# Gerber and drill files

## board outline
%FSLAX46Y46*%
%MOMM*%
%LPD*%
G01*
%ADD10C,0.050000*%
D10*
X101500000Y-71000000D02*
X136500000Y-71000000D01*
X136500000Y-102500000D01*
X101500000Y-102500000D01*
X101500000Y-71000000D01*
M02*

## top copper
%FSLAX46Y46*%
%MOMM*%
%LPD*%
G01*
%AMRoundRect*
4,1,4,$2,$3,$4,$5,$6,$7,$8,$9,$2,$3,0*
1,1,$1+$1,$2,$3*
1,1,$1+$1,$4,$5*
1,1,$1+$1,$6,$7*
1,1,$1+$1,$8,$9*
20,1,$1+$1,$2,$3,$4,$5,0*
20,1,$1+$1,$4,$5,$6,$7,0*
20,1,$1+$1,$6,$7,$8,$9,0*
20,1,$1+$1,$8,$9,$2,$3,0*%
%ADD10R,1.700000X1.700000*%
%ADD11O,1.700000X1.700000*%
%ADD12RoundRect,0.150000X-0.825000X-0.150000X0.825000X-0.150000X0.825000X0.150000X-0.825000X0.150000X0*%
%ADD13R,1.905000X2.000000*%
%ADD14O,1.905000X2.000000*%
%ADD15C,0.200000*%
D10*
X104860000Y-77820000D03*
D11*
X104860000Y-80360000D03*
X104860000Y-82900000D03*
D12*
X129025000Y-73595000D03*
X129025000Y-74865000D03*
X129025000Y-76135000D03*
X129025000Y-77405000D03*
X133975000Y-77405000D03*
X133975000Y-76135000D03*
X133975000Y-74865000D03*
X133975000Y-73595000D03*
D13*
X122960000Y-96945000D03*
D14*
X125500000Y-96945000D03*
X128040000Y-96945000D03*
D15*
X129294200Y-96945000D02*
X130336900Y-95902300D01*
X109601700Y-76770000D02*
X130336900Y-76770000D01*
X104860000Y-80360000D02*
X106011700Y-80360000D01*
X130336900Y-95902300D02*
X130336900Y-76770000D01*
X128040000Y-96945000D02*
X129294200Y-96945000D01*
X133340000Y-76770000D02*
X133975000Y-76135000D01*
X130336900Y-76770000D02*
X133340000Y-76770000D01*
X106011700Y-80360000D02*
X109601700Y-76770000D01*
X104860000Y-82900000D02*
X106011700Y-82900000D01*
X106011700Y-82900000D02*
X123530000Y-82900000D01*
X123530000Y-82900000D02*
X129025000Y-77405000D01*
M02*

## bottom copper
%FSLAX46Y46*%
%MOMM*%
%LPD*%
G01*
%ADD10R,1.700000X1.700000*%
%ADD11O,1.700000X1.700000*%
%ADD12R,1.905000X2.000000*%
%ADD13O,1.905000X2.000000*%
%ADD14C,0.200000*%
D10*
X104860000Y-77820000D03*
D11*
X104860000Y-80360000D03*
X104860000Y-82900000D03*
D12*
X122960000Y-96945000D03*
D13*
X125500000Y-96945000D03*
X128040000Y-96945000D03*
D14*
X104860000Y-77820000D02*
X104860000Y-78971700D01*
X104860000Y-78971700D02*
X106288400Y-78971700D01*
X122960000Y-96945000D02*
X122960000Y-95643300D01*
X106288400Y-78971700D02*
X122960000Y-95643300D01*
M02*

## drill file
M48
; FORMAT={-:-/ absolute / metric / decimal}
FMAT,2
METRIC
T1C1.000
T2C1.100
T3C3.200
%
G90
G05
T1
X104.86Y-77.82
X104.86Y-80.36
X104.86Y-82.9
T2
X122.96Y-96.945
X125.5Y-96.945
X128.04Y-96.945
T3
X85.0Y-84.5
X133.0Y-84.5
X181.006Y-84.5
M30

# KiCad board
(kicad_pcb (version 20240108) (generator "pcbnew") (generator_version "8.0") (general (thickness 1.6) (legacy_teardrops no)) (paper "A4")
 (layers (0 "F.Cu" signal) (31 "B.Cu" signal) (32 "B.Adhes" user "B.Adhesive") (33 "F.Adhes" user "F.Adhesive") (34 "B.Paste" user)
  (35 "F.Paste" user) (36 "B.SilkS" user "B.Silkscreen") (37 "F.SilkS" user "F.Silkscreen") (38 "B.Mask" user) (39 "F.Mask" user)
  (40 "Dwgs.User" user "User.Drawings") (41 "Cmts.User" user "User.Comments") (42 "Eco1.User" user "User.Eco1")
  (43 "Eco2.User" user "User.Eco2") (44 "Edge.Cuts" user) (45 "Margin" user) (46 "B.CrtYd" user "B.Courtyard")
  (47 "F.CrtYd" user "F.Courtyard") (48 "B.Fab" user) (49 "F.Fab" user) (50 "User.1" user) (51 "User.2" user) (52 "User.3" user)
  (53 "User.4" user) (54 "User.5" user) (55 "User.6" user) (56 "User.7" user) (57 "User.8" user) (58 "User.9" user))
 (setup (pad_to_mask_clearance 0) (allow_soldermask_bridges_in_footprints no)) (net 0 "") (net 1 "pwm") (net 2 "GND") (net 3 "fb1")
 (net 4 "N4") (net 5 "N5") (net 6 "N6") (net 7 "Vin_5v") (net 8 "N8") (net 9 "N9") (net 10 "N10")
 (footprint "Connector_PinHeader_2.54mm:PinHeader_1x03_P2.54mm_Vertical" (layer "F.Cu") (at 104.86 77.82)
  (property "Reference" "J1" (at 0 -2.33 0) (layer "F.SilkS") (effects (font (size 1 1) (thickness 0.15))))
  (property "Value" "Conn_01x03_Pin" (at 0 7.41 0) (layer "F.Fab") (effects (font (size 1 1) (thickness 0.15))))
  (pad "1" thru_hole rect (at 0 0) (size 1.7 1.7) (drill 1) (layers "*.Cu" "*.Mask") (remove_unused_layers no) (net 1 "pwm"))
  (pad "2" thru_hole oval (at 0 2.54) (size 1.7 1.7) (drill 1) (layers "*.Cu" "*.Mask") (remove_unused_layers no) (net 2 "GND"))
  (pad "3" thru_hole oval (at 0 5.08) (size 1.7 1.7) (drill 1) (layers "*.Cu" "*.Mask") (remove_unused_layers no) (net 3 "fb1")))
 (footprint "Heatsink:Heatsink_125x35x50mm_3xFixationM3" (layer "F.Cu") (at 133 84.5)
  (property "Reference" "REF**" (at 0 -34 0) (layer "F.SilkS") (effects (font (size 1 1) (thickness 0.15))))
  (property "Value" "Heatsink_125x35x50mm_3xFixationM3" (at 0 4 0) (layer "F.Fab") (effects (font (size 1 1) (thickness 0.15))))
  (pad "" np_thru_hole circle (at -48 0) (size 3.2 3.2) (drill 3.2) (layers "*.Cu" "*.SilkS" "*.Mask"))
  (pad "" np_thru_hole circle (at 0 0) (size 3.2 3.2) (drill 3.2) (layers "*.Cu" "*.SilkS" "*.Mask"))
  (pad "" np_thru_hole circle (at 48.006 0) (size 3.2 3.2) (drill 3.2) (layers "*.Cu" "*.SilkS" "*.Mask")))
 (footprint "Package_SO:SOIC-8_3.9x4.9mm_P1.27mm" (layer "F.Cu") (at 131.5 75.5)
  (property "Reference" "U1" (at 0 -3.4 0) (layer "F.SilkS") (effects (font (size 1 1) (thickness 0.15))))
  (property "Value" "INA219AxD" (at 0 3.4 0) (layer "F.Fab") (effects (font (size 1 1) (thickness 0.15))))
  (pad "1" smd roundrect (at -2.475 -1.905) (size 1.95 0.6) (layers "F.Cu" "F.Paste" "F.Mask") (roundrect_rratio 0.25) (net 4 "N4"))
  (pad "2" smd roundrect (at -2.475 -0.635) (size 1.95 0.6) (layers "F.Cu" "F.Paste" "F.Mask") (roundrect_rratio 0.25) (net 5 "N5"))
  (pad "3" smd roundrect (at -2.475 0.635) (size 1.95 0.6) (layers "F.Cu" "F.Paste" "F.Mask") (roundrect_rratio 0.25) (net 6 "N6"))
  (pad "4" smd roundrect (at -2.475 1.905) (size 1.95 0.6) (layers "F.Cu" "F.Paste" "F.Mask") (roundrect_rratio 0.25) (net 3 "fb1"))
  (pad "5" smd roundrect (at 2.475 1.905) (size 1.95 0.6) (layers "F.Cu" "F.Paste" "F.Mask") (roundrect_rratio 0.25) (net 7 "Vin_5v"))
  (pad "6" smd roundrect (at 2.475 0.635) (size 1.95 0.6) (layers "F.Cu" "F.Paste" "F.Mask") (roundrect_rratio 0.25) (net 2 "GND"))
  (pad "7" smd roundrect (at 2.475 -0.635) (size 1.95 0.6) (layers "F.Cu" "F.Paste" "F.Mask") (roundrect_rratio 0.25) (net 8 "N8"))
  (pad "8" smd roundrect (at 2.475 -1.905) (size 1.95 0.6) (layers "F.Cu" "F.Paste" "F.Mask") (roundrect_rratio 0.25) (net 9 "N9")))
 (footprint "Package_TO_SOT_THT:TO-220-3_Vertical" (layer "F.Cu") (at 122.96 96.945)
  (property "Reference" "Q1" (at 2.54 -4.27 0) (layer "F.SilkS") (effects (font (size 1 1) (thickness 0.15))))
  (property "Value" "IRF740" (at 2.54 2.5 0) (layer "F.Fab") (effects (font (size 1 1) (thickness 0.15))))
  (pad "1" thru_hole rect (at 0 0) (size 1.905 2) (drill 1.1) (layers "*.Cu" "*.Mask") (remove_unused_layers no) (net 1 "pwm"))
  (pad "2" thru_hole oval (at 2.54 0) (size 1.905 2) (drill 1.1) (layers "*.Cu" "*.Mask") (remove_unused_layers no) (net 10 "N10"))
  (pad "3" thru_hole oval (at 5.08 0) (size 1.905 2) (drill 1.1) (layers "*.Cu" "*.Mask") (remove_unused_layers no) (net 2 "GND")))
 (gr_rect (start 101.5 71) (end 136.5 102.5) (stroke (width 0.05) (type default)) (fill none) (layer "Edge.Cuts"))
 (segment (start 104.86 77.82) (end 104.86 78.9717) (width 0.2) (layer "B.Cu") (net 1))
 (segment (start 104.86 78.9717) (end 106.2884 78.9717) (width 0.2) (layer "B.Cu") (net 1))
 (segment (start 122.96 96.945) (end 122.96 95.6433) (width 0.2) (layer "B.Cu") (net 1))
 (segment (start 106.2884 78.9717) (end 122.96 95.6433) (width 0.2) (layer "B.Cu") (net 1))
 (segment (start 129.2942 96.945) (end 130.3369 95.9023) (width 0.2) (layer "F.Cu") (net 2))
 (segment (start 109.6017 76.77) (end 130.3369 76.77) (width 0.2) (layer "F.Cu") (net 2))
 (segment (start 104.86 80.36) (end 106.0117 80.36) (width 0.2) (layer "F.Cu") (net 2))
 (segment (start 130.3369 95.9023) (end 130.3369 76.77) (width 0.2) (layer "F.Cu") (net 2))
 (segment (start 128.04 96.945) (end 129.2942 96.945) (width 0.2) (layer "F.Cu") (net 2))
 (segment (start 133.34 76.77) (end 133.975 76.135) (width 0.2) (layer "F.Cu") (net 2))
 (segment (start 130.3369 76.77) (end 133.34 76.77) (width 0.2) (layer "F.Cu") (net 2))
 (segment (start 106.0117 80.36) (end 109.6017 76.77) (width 0.2) (layer "F.Cu") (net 2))
 (segment (start 104.86 82.9) (end 106.0117 82.9) (width 0.2) (layer "F.Cu") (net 3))
 (segment (start 106.0117 82.9) (end 123.53 82.9) (width 0.2) (layer "F.Cu") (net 3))
 (segment (start 123.53 82.9) (end 129.025 77.405) (width 0.2) (layer "F.Cu") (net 3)))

